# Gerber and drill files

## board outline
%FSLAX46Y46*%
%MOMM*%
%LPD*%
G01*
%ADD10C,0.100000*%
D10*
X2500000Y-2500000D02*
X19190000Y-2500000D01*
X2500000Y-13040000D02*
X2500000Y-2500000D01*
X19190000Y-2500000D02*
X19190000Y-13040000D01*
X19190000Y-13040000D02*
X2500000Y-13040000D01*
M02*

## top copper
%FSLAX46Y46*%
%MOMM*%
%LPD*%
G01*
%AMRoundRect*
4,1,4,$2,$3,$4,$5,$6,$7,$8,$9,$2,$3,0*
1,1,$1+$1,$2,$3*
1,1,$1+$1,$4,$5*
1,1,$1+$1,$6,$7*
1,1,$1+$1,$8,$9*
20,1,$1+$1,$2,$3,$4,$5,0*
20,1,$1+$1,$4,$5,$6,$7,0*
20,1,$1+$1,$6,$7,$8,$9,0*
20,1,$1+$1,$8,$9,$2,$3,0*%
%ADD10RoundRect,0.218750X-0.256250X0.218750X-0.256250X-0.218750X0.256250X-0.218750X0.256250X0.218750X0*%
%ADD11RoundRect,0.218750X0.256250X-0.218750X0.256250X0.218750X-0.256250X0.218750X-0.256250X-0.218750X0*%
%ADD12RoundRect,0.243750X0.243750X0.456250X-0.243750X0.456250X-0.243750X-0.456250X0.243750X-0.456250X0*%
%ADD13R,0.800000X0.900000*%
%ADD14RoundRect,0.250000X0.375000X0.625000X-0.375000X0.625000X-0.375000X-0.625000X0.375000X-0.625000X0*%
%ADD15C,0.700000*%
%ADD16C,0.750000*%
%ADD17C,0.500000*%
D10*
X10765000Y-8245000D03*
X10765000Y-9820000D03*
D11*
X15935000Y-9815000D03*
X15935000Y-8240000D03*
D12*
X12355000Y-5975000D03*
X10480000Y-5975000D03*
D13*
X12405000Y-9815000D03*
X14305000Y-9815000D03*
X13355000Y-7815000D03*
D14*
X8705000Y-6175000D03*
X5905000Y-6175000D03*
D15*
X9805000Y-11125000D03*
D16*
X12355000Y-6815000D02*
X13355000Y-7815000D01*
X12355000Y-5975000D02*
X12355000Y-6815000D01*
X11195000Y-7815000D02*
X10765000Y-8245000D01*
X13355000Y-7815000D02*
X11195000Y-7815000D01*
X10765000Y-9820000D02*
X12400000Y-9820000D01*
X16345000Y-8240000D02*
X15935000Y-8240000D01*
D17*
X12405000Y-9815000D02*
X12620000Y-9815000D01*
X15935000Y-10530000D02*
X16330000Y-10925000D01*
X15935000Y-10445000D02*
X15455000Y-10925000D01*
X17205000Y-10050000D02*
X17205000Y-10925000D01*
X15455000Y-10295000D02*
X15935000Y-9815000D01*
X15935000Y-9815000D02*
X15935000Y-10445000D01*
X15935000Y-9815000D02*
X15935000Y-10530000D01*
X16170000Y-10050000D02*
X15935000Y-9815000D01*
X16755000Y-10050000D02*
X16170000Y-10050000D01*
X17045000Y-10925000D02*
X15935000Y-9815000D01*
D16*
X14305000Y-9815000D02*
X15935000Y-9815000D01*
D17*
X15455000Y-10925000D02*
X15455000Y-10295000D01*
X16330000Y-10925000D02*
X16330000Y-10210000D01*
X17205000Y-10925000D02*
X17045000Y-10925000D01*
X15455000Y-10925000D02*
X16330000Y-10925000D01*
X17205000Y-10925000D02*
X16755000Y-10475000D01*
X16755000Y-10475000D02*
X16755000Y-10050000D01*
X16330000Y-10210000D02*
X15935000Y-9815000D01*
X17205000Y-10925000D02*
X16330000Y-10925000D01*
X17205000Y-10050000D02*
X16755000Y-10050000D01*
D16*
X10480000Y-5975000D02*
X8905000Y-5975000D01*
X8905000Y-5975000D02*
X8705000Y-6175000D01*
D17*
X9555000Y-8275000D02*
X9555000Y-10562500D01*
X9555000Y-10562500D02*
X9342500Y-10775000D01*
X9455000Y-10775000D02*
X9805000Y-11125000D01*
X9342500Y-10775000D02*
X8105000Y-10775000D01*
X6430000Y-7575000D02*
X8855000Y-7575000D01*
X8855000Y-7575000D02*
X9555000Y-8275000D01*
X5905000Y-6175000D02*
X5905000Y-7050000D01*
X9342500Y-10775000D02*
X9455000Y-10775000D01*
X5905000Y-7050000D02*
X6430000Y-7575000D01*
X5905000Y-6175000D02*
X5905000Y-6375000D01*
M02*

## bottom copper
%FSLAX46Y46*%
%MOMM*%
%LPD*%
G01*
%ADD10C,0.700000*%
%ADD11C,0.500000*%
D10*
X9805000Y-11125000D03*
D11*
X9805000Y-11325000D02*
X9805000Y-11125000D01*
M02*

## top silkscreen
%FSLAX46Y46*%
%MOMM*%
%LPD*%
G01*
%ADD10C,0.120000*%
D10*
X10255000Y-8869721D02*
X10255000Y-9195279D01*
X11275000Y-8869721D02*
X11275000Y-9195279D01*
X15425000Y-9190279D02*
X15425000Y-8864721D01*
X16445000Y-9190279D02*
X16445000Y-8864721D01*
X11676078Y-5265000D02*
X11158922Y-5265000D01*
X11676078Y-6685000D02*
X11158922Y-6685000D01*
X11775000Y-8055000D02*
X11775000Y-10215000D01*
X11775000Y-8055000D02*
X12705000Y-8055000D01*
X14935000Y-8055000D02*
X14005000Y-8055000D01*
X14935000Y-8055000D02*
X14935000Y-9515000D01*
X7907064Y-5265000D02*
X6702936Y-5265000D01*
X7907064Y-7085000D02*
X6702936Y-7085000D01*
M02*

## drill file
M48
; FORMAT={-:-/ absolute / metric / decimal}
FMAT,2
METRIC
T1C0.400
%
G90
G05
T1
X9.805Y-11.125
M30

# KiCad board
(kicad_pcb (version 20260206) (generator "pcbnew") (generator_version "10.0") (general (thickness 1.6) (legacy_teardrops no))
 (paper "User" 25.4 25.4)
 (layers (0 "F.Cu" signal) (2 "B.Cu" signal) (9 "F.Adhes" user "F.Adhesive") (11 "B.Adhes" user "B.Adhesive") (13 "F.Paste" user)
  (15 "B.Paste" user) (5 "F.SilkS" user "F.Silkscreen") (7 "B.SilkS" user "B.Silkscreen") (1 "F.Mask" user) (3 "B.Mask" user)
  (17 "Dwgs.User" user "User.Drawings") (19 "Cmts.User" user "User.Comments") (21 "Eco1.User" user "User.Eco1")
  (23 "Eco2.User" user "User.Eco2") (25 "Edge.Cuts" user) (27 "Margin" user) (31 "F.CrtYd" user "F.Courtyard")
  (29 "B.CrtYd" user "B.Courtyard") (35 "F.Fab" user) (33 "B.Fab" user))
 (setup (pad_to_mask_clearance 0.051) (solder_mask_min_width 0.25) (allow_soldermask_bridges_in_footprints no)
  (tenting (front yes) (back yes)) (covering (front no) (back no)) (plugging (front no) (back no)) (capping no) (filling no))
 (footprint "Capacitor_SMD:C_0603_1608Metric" (layer "F.Cu") (at 10.765 9.0325 -90)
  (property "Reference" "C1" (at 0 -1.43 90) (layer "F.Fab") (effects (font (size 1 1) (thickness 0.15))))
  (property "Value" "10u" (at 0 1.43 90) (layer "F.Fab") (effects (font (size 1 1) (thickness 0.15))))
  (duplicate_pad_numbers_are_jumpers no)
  (fp_line (start -0.162779 0.51) (end 0.162779 0.51) (stroke (width 0.12) (type solid)) (layer "F.SilkS"))
  (fp_line (start -0.162779 -0.51) (end 0.162779 -0.51) (stroke (width 0.12) (type solid)) (layer "F.SilkS"))
  (pad "1" smd roundrect (at -0.7875 0 270) (size 0.875 0.95) (layers "F.Cu" "F.Mask" "F.Paste") (roundrect_rratio 0.25)
   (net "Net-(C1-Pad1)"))
  (pad "2" smd roundrect (at 0.7875 0 270) (size 0.875 0.95) (layers "F.Cu" "F.Mask" "F.Paste") (roundrect_rratio 0.25) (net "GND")))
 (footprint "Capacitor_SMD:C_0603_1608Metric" (layer "F.Cu") (at 15.935 9.0275 90)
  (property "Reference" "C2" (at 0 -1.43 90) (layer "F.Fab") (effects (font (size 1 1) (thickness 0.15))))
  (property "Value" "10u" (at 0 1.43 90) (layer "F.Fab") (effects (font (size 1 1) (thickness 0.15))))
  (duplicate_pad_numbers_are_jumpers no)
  (fp_line (start -0.162779 -0.51) (end 0.162779 -0.51) (stroke (width 0.12) (type solid)) (layer "F.SilkS"))
  (fp_line (start -0.162779 0.51) (end 0.162779 0.51) (stroke (width 0.12) (type solid)) (layer "F.SilkS"))
  (pad "1" smd roundrect (at -0.7875 0 90) (size 0.875 0.95) (layers "F.Cu" "F.Mask" "F.Paste") (roundrect_rratio 0.25) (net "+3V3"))
  (pad "2" smd roundrect (at 0.7875 0 90) (size 0.875 0.95) (layers "F.Cu" "F.Mask" "F.Paste") (roundrect_rratio 0.25) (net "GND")))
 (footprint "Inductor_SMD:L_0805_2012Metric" (layer "F.Cu") (at 11.4175 5.975 180)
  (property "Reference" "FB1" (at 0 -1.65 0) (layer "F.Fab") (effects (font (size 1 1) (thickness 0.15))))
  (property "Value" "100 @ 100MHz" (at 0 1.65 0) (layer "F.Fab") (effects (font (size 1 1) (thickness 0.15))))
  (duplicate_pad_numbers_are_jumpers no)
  (fp_line (start -0.258578 0.71) (end 0.258578 0.71) (stroke (width 0.12) (type solid)) (layer "F.SilkS"))
  (fp_line (start -0.258578 -0.71) (end 0.258578 -0.71) (stroke (width 0.12) (type solid)) (layer "F.SilkS"))
  (pad "1" smd roundrect (at -0.9375 0 180) (size 0.975 1.4) (layers "F.Cu" "F.Mask" "F.Paste") (roundrect_rratio 0.25)
   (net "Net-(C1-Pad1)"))
  (pad "2" smd roundrect (at 0.9375 0 180) (size 0.975 1.4) (layers "F.Cu" "F.Mask" "F.Paste") (roundrect_rratio 0.25) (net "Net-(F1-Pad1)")))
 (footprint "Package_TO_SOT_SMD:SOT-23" (layer "F.Cu") (at 13.355 8.815 90)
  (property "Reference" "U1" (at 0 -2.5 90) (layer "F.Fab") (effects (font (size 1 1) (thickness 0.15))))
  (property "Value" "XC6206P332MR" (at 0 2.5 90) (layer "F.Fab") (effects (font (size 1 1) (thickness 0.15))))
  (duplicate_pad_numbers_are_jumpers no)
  (fp_line (start 0.76 -1.58) (end -1.4 -1.58) (stroke (width 0.12) (type solid)) (layer "F.SilkS"))
  (fp_line (start 0.76 -1.58) (end 0.76 -0.65) (stroke (width 0.12) (type solid)) (layer "F.SilkS"))
  (fp_line (start 0.76 1.58) (end 0.76 0.65) (stroke (width 0.12) (type solid)) (layer "F.SilkS"))
  (fp_line (start 0.76 1.58) (end -0.7 1.58) (stroke (width 0.12) (type solid)) (layer "F.SilkS"))
  (pad "1" smd rect (at -1 -0.95 90) (size 0.9 0.8) (layers "F.Cu" "F.Mask" "F.Paste") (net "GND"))
  (pad "2" smd rect (at -1 0.95 90) (size 0.9 0.8) (layers "F.Cu" "F.Mask" "F.Paste") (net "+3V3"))
  (pad "3" smd rect (at 1 0 90) (size 0.9 0.8) (layers "F.Cu" "F.Mask" "F.Paste") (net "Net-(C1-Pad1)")))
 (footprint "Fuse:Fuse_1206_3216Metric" (layer "F.Cu") (at 7.305 6.175 180)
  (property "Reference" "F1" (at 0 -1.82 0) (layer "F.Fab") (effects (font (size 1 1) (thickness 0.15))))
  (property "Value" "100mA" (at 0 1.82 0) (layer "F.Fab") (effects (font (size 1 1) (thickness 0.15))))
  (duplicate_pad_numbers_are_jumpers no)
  (fp_line (start -0.602064 0.91) (end 0.602064 0.91) (stroke (width 0.12) (type solid)) (layer "F.SilkS"))
  (fp_line (start -0.602064 -0.91) (end 0.602064 -0.91) (stroke (width 0.12) (type solid)) (layer "F.SilkS"))
  (pad "1" smd roundrect (at -1.4 0 180) (size 1.25 1.75) (layers "F.Cu" "F.Mask" "F.Paste") (roundrect_rratio 0.2) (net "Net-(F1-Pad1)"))
  (pad "2" smd roundrect (at 1.4 0 180) (size 1.25 1.75) (layers "F.Cu" "F.Mask" "F.Paste") (roundrect_rratio 0.2) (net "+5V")))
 (gr_line (start 2.5 2.5) (end 19.19 2.5) (stroke (width 0.1) (type default)) (layer "Edge.Cuts"))
 (gr_line (start 2.5 13.04) (end 2.5 2.5) (stroke (width 0.1) (type default)) (layer "Edge.Cuts"))
 (gr_line (start 19.19 2.5) (end 19.19 13.04) (stroke (width 0.1) (type default)) (layer "Edge.Cuts"))
 (gr_line (start 19.19 13.04) (end 2.5 13.04) (stroke (width 0.1) (type default)) (layer "Edge.Cuts"))
 (segment (start 12.355 6.815) (end 13.355 7.815) (width 0.75) (layer "F.Cu") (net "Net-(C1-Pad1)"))
 (segment (start 12.355 5.975) (end 12.355 6.815) (width 0.75) (layer "F.Cu") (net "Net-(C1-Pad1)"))
 (segment (start 11.195 7.815) (end 10.765 8.245) (width 0.75) (layer "F.Cu") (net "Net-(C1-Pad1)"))
 (segment (start 13.355 7.815) (end 11.195 7.815) (width 0.75) (layer "F.Cu") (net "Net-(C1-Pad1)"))
 (segment (start 10.765 9.82) (end 12.4 9.82) (width 0.75) (layer "F.Cu") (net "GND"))
 (segment (start 16.345 8.24) (end 15.935 8.24) (width 0.75) (layer "F.Cu") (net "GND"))
 (segment (start 12.405 9.815) (end 12.62 9.815) (width 0.5) (layer "F.Cu") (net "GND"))
 (segment (start 15.935 10.53) (end 16.33 10.925) (width 0.5) (layer "F.Cu") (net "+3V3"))
 (segment (start 15.935 10.445) (end 15.455 10.925) (width 0.5) (layer "F.Cu") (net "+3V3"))
 (segment (start 17.205 10.05) (end 17.205 10.925) (width 0.5) (layer "F.Cu") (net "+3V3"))
 (segment (start 15.455 10.295) (end 15.935 9.815) (width 0.5) (layer "F.Cu") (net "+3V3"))
 (segment (start 15.935 9.815) (end 15.935 10.445) (width 0.5) (layer "F.Cu") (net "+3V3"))
 (segment (start 15.935 9.815) (end 15.935 10.53) (width 0.5) (layer "F.Cu") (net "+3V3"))
 (segment (start 16.17 10.05) (end 15.935 9.815) (width 0.5) (layer "F.Cu") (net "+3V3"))
 (segment (start 16.755 10.05) (end 16.17 10.05) (width 0.5) (layer "F.Cu") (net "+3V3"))
 (segment (start 17.045 10.925) (end 15.935 9.815) (width 0.5) (layer "F.Cu") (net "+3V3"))
 (segment (start 14.305 9.815) (end 15.935 9.815) (width 0.75) (layer "F.Cu") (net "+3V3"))
 (segment (start 15.455 10.925) (end 15.455 10.295) (width 0.5) (layer "F.Cu") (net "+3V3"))
 (segment (start 16.33 10.925) (end 16.33 10.21) (width 0.5) (layer "F.Cu") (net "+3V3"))
 (segment (start 17.205 10.925) (end 17.045 10.925) (width 0.5) (layer "F.Cu") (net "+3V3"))
 (segment (start 15.455 10.925) (end 16.33 10.925) (width 0.5) (layer "F.Cu") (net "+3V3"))
 (segment (start 17.205 10.925) (end 16.755 10.475) (width 0.5) (layer "F.Cu") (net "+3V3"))
 (segment (start 16.755 10.475) (end 16.755 10.05) (width 0.5) (layer "F.Cu") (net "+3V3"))
 (segment (start 16.33 10.21) (end 15.935 9.815) (width 0.5) (layer "F.Cu") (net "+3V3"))
 (segment (start 17.205 10.925) (end 16.33 10.925) (width 0.5) (layer "F.Cu") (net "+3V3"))
 (segment (start 17.205 10.05) (end 16.755 10.05) (width 0.5) (layer "F.Cu") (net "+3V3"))
 (segment (start 10.48 5.975) (end 8.905 5.975) (width 0.75) (layer "F.Cu") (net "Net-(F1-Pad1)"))
 (segment (start 8.905 5.975) (end 8.705 6.175) (width 0.75) (layer "F.Cu") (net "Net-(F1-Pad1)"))
 (segment (start 9.555 8.275) (end 9.555 10.5625) (width 0.5) (layer "F.Cu") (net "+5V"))
 (segment (start 9.555 10.5625) (end 9.3425 10.775) (width 0.5) (layer "F.Cu") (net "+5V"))
 (segment (start 9.455 10.775) (end 9.805 11.125) (width 0.5) (layer "F.Cu") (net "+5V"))
 (segment (start 9.3425 10.775) (end 8.105 10.775) (width 0.5) (layer "F.Cu") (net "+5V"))
 (segment (start 6.43 7.575) (end 8.855 7.575) (width 0.5) (layer "F.Cu") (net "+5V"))
 (segment (start 8.855 7.575) (end 9.555 8.275) (width 0.5) (layer "F.Cu") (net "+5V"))
 (segment (start 5.905 6.175) (end 5.905 7.05) (width 0.5) (layer "F.Cu") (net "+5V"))
 (segment (start 9.3425 10.775) (end 9.455 10.775) (width 0.5) (layer "F.Cu") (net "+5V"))
 (segment (start 5.905 7.05) (end 6.43 7.575) (width 0.5) (layer "F.Cu") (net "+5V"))
 (segment (start 5.905 6.175) (end 5.905 6.375) (width 0.5) (layer "F.Cu") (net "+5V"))
 (via (at 9.805 11.125) (size 0.7) (drill 0.4) (layers "F.Cu" "B.Cu") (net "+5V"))
 (segment (start 9.805 11.325) (end 9.805 11.125) (width 0.5) (layer "B.Cu") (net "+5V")))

